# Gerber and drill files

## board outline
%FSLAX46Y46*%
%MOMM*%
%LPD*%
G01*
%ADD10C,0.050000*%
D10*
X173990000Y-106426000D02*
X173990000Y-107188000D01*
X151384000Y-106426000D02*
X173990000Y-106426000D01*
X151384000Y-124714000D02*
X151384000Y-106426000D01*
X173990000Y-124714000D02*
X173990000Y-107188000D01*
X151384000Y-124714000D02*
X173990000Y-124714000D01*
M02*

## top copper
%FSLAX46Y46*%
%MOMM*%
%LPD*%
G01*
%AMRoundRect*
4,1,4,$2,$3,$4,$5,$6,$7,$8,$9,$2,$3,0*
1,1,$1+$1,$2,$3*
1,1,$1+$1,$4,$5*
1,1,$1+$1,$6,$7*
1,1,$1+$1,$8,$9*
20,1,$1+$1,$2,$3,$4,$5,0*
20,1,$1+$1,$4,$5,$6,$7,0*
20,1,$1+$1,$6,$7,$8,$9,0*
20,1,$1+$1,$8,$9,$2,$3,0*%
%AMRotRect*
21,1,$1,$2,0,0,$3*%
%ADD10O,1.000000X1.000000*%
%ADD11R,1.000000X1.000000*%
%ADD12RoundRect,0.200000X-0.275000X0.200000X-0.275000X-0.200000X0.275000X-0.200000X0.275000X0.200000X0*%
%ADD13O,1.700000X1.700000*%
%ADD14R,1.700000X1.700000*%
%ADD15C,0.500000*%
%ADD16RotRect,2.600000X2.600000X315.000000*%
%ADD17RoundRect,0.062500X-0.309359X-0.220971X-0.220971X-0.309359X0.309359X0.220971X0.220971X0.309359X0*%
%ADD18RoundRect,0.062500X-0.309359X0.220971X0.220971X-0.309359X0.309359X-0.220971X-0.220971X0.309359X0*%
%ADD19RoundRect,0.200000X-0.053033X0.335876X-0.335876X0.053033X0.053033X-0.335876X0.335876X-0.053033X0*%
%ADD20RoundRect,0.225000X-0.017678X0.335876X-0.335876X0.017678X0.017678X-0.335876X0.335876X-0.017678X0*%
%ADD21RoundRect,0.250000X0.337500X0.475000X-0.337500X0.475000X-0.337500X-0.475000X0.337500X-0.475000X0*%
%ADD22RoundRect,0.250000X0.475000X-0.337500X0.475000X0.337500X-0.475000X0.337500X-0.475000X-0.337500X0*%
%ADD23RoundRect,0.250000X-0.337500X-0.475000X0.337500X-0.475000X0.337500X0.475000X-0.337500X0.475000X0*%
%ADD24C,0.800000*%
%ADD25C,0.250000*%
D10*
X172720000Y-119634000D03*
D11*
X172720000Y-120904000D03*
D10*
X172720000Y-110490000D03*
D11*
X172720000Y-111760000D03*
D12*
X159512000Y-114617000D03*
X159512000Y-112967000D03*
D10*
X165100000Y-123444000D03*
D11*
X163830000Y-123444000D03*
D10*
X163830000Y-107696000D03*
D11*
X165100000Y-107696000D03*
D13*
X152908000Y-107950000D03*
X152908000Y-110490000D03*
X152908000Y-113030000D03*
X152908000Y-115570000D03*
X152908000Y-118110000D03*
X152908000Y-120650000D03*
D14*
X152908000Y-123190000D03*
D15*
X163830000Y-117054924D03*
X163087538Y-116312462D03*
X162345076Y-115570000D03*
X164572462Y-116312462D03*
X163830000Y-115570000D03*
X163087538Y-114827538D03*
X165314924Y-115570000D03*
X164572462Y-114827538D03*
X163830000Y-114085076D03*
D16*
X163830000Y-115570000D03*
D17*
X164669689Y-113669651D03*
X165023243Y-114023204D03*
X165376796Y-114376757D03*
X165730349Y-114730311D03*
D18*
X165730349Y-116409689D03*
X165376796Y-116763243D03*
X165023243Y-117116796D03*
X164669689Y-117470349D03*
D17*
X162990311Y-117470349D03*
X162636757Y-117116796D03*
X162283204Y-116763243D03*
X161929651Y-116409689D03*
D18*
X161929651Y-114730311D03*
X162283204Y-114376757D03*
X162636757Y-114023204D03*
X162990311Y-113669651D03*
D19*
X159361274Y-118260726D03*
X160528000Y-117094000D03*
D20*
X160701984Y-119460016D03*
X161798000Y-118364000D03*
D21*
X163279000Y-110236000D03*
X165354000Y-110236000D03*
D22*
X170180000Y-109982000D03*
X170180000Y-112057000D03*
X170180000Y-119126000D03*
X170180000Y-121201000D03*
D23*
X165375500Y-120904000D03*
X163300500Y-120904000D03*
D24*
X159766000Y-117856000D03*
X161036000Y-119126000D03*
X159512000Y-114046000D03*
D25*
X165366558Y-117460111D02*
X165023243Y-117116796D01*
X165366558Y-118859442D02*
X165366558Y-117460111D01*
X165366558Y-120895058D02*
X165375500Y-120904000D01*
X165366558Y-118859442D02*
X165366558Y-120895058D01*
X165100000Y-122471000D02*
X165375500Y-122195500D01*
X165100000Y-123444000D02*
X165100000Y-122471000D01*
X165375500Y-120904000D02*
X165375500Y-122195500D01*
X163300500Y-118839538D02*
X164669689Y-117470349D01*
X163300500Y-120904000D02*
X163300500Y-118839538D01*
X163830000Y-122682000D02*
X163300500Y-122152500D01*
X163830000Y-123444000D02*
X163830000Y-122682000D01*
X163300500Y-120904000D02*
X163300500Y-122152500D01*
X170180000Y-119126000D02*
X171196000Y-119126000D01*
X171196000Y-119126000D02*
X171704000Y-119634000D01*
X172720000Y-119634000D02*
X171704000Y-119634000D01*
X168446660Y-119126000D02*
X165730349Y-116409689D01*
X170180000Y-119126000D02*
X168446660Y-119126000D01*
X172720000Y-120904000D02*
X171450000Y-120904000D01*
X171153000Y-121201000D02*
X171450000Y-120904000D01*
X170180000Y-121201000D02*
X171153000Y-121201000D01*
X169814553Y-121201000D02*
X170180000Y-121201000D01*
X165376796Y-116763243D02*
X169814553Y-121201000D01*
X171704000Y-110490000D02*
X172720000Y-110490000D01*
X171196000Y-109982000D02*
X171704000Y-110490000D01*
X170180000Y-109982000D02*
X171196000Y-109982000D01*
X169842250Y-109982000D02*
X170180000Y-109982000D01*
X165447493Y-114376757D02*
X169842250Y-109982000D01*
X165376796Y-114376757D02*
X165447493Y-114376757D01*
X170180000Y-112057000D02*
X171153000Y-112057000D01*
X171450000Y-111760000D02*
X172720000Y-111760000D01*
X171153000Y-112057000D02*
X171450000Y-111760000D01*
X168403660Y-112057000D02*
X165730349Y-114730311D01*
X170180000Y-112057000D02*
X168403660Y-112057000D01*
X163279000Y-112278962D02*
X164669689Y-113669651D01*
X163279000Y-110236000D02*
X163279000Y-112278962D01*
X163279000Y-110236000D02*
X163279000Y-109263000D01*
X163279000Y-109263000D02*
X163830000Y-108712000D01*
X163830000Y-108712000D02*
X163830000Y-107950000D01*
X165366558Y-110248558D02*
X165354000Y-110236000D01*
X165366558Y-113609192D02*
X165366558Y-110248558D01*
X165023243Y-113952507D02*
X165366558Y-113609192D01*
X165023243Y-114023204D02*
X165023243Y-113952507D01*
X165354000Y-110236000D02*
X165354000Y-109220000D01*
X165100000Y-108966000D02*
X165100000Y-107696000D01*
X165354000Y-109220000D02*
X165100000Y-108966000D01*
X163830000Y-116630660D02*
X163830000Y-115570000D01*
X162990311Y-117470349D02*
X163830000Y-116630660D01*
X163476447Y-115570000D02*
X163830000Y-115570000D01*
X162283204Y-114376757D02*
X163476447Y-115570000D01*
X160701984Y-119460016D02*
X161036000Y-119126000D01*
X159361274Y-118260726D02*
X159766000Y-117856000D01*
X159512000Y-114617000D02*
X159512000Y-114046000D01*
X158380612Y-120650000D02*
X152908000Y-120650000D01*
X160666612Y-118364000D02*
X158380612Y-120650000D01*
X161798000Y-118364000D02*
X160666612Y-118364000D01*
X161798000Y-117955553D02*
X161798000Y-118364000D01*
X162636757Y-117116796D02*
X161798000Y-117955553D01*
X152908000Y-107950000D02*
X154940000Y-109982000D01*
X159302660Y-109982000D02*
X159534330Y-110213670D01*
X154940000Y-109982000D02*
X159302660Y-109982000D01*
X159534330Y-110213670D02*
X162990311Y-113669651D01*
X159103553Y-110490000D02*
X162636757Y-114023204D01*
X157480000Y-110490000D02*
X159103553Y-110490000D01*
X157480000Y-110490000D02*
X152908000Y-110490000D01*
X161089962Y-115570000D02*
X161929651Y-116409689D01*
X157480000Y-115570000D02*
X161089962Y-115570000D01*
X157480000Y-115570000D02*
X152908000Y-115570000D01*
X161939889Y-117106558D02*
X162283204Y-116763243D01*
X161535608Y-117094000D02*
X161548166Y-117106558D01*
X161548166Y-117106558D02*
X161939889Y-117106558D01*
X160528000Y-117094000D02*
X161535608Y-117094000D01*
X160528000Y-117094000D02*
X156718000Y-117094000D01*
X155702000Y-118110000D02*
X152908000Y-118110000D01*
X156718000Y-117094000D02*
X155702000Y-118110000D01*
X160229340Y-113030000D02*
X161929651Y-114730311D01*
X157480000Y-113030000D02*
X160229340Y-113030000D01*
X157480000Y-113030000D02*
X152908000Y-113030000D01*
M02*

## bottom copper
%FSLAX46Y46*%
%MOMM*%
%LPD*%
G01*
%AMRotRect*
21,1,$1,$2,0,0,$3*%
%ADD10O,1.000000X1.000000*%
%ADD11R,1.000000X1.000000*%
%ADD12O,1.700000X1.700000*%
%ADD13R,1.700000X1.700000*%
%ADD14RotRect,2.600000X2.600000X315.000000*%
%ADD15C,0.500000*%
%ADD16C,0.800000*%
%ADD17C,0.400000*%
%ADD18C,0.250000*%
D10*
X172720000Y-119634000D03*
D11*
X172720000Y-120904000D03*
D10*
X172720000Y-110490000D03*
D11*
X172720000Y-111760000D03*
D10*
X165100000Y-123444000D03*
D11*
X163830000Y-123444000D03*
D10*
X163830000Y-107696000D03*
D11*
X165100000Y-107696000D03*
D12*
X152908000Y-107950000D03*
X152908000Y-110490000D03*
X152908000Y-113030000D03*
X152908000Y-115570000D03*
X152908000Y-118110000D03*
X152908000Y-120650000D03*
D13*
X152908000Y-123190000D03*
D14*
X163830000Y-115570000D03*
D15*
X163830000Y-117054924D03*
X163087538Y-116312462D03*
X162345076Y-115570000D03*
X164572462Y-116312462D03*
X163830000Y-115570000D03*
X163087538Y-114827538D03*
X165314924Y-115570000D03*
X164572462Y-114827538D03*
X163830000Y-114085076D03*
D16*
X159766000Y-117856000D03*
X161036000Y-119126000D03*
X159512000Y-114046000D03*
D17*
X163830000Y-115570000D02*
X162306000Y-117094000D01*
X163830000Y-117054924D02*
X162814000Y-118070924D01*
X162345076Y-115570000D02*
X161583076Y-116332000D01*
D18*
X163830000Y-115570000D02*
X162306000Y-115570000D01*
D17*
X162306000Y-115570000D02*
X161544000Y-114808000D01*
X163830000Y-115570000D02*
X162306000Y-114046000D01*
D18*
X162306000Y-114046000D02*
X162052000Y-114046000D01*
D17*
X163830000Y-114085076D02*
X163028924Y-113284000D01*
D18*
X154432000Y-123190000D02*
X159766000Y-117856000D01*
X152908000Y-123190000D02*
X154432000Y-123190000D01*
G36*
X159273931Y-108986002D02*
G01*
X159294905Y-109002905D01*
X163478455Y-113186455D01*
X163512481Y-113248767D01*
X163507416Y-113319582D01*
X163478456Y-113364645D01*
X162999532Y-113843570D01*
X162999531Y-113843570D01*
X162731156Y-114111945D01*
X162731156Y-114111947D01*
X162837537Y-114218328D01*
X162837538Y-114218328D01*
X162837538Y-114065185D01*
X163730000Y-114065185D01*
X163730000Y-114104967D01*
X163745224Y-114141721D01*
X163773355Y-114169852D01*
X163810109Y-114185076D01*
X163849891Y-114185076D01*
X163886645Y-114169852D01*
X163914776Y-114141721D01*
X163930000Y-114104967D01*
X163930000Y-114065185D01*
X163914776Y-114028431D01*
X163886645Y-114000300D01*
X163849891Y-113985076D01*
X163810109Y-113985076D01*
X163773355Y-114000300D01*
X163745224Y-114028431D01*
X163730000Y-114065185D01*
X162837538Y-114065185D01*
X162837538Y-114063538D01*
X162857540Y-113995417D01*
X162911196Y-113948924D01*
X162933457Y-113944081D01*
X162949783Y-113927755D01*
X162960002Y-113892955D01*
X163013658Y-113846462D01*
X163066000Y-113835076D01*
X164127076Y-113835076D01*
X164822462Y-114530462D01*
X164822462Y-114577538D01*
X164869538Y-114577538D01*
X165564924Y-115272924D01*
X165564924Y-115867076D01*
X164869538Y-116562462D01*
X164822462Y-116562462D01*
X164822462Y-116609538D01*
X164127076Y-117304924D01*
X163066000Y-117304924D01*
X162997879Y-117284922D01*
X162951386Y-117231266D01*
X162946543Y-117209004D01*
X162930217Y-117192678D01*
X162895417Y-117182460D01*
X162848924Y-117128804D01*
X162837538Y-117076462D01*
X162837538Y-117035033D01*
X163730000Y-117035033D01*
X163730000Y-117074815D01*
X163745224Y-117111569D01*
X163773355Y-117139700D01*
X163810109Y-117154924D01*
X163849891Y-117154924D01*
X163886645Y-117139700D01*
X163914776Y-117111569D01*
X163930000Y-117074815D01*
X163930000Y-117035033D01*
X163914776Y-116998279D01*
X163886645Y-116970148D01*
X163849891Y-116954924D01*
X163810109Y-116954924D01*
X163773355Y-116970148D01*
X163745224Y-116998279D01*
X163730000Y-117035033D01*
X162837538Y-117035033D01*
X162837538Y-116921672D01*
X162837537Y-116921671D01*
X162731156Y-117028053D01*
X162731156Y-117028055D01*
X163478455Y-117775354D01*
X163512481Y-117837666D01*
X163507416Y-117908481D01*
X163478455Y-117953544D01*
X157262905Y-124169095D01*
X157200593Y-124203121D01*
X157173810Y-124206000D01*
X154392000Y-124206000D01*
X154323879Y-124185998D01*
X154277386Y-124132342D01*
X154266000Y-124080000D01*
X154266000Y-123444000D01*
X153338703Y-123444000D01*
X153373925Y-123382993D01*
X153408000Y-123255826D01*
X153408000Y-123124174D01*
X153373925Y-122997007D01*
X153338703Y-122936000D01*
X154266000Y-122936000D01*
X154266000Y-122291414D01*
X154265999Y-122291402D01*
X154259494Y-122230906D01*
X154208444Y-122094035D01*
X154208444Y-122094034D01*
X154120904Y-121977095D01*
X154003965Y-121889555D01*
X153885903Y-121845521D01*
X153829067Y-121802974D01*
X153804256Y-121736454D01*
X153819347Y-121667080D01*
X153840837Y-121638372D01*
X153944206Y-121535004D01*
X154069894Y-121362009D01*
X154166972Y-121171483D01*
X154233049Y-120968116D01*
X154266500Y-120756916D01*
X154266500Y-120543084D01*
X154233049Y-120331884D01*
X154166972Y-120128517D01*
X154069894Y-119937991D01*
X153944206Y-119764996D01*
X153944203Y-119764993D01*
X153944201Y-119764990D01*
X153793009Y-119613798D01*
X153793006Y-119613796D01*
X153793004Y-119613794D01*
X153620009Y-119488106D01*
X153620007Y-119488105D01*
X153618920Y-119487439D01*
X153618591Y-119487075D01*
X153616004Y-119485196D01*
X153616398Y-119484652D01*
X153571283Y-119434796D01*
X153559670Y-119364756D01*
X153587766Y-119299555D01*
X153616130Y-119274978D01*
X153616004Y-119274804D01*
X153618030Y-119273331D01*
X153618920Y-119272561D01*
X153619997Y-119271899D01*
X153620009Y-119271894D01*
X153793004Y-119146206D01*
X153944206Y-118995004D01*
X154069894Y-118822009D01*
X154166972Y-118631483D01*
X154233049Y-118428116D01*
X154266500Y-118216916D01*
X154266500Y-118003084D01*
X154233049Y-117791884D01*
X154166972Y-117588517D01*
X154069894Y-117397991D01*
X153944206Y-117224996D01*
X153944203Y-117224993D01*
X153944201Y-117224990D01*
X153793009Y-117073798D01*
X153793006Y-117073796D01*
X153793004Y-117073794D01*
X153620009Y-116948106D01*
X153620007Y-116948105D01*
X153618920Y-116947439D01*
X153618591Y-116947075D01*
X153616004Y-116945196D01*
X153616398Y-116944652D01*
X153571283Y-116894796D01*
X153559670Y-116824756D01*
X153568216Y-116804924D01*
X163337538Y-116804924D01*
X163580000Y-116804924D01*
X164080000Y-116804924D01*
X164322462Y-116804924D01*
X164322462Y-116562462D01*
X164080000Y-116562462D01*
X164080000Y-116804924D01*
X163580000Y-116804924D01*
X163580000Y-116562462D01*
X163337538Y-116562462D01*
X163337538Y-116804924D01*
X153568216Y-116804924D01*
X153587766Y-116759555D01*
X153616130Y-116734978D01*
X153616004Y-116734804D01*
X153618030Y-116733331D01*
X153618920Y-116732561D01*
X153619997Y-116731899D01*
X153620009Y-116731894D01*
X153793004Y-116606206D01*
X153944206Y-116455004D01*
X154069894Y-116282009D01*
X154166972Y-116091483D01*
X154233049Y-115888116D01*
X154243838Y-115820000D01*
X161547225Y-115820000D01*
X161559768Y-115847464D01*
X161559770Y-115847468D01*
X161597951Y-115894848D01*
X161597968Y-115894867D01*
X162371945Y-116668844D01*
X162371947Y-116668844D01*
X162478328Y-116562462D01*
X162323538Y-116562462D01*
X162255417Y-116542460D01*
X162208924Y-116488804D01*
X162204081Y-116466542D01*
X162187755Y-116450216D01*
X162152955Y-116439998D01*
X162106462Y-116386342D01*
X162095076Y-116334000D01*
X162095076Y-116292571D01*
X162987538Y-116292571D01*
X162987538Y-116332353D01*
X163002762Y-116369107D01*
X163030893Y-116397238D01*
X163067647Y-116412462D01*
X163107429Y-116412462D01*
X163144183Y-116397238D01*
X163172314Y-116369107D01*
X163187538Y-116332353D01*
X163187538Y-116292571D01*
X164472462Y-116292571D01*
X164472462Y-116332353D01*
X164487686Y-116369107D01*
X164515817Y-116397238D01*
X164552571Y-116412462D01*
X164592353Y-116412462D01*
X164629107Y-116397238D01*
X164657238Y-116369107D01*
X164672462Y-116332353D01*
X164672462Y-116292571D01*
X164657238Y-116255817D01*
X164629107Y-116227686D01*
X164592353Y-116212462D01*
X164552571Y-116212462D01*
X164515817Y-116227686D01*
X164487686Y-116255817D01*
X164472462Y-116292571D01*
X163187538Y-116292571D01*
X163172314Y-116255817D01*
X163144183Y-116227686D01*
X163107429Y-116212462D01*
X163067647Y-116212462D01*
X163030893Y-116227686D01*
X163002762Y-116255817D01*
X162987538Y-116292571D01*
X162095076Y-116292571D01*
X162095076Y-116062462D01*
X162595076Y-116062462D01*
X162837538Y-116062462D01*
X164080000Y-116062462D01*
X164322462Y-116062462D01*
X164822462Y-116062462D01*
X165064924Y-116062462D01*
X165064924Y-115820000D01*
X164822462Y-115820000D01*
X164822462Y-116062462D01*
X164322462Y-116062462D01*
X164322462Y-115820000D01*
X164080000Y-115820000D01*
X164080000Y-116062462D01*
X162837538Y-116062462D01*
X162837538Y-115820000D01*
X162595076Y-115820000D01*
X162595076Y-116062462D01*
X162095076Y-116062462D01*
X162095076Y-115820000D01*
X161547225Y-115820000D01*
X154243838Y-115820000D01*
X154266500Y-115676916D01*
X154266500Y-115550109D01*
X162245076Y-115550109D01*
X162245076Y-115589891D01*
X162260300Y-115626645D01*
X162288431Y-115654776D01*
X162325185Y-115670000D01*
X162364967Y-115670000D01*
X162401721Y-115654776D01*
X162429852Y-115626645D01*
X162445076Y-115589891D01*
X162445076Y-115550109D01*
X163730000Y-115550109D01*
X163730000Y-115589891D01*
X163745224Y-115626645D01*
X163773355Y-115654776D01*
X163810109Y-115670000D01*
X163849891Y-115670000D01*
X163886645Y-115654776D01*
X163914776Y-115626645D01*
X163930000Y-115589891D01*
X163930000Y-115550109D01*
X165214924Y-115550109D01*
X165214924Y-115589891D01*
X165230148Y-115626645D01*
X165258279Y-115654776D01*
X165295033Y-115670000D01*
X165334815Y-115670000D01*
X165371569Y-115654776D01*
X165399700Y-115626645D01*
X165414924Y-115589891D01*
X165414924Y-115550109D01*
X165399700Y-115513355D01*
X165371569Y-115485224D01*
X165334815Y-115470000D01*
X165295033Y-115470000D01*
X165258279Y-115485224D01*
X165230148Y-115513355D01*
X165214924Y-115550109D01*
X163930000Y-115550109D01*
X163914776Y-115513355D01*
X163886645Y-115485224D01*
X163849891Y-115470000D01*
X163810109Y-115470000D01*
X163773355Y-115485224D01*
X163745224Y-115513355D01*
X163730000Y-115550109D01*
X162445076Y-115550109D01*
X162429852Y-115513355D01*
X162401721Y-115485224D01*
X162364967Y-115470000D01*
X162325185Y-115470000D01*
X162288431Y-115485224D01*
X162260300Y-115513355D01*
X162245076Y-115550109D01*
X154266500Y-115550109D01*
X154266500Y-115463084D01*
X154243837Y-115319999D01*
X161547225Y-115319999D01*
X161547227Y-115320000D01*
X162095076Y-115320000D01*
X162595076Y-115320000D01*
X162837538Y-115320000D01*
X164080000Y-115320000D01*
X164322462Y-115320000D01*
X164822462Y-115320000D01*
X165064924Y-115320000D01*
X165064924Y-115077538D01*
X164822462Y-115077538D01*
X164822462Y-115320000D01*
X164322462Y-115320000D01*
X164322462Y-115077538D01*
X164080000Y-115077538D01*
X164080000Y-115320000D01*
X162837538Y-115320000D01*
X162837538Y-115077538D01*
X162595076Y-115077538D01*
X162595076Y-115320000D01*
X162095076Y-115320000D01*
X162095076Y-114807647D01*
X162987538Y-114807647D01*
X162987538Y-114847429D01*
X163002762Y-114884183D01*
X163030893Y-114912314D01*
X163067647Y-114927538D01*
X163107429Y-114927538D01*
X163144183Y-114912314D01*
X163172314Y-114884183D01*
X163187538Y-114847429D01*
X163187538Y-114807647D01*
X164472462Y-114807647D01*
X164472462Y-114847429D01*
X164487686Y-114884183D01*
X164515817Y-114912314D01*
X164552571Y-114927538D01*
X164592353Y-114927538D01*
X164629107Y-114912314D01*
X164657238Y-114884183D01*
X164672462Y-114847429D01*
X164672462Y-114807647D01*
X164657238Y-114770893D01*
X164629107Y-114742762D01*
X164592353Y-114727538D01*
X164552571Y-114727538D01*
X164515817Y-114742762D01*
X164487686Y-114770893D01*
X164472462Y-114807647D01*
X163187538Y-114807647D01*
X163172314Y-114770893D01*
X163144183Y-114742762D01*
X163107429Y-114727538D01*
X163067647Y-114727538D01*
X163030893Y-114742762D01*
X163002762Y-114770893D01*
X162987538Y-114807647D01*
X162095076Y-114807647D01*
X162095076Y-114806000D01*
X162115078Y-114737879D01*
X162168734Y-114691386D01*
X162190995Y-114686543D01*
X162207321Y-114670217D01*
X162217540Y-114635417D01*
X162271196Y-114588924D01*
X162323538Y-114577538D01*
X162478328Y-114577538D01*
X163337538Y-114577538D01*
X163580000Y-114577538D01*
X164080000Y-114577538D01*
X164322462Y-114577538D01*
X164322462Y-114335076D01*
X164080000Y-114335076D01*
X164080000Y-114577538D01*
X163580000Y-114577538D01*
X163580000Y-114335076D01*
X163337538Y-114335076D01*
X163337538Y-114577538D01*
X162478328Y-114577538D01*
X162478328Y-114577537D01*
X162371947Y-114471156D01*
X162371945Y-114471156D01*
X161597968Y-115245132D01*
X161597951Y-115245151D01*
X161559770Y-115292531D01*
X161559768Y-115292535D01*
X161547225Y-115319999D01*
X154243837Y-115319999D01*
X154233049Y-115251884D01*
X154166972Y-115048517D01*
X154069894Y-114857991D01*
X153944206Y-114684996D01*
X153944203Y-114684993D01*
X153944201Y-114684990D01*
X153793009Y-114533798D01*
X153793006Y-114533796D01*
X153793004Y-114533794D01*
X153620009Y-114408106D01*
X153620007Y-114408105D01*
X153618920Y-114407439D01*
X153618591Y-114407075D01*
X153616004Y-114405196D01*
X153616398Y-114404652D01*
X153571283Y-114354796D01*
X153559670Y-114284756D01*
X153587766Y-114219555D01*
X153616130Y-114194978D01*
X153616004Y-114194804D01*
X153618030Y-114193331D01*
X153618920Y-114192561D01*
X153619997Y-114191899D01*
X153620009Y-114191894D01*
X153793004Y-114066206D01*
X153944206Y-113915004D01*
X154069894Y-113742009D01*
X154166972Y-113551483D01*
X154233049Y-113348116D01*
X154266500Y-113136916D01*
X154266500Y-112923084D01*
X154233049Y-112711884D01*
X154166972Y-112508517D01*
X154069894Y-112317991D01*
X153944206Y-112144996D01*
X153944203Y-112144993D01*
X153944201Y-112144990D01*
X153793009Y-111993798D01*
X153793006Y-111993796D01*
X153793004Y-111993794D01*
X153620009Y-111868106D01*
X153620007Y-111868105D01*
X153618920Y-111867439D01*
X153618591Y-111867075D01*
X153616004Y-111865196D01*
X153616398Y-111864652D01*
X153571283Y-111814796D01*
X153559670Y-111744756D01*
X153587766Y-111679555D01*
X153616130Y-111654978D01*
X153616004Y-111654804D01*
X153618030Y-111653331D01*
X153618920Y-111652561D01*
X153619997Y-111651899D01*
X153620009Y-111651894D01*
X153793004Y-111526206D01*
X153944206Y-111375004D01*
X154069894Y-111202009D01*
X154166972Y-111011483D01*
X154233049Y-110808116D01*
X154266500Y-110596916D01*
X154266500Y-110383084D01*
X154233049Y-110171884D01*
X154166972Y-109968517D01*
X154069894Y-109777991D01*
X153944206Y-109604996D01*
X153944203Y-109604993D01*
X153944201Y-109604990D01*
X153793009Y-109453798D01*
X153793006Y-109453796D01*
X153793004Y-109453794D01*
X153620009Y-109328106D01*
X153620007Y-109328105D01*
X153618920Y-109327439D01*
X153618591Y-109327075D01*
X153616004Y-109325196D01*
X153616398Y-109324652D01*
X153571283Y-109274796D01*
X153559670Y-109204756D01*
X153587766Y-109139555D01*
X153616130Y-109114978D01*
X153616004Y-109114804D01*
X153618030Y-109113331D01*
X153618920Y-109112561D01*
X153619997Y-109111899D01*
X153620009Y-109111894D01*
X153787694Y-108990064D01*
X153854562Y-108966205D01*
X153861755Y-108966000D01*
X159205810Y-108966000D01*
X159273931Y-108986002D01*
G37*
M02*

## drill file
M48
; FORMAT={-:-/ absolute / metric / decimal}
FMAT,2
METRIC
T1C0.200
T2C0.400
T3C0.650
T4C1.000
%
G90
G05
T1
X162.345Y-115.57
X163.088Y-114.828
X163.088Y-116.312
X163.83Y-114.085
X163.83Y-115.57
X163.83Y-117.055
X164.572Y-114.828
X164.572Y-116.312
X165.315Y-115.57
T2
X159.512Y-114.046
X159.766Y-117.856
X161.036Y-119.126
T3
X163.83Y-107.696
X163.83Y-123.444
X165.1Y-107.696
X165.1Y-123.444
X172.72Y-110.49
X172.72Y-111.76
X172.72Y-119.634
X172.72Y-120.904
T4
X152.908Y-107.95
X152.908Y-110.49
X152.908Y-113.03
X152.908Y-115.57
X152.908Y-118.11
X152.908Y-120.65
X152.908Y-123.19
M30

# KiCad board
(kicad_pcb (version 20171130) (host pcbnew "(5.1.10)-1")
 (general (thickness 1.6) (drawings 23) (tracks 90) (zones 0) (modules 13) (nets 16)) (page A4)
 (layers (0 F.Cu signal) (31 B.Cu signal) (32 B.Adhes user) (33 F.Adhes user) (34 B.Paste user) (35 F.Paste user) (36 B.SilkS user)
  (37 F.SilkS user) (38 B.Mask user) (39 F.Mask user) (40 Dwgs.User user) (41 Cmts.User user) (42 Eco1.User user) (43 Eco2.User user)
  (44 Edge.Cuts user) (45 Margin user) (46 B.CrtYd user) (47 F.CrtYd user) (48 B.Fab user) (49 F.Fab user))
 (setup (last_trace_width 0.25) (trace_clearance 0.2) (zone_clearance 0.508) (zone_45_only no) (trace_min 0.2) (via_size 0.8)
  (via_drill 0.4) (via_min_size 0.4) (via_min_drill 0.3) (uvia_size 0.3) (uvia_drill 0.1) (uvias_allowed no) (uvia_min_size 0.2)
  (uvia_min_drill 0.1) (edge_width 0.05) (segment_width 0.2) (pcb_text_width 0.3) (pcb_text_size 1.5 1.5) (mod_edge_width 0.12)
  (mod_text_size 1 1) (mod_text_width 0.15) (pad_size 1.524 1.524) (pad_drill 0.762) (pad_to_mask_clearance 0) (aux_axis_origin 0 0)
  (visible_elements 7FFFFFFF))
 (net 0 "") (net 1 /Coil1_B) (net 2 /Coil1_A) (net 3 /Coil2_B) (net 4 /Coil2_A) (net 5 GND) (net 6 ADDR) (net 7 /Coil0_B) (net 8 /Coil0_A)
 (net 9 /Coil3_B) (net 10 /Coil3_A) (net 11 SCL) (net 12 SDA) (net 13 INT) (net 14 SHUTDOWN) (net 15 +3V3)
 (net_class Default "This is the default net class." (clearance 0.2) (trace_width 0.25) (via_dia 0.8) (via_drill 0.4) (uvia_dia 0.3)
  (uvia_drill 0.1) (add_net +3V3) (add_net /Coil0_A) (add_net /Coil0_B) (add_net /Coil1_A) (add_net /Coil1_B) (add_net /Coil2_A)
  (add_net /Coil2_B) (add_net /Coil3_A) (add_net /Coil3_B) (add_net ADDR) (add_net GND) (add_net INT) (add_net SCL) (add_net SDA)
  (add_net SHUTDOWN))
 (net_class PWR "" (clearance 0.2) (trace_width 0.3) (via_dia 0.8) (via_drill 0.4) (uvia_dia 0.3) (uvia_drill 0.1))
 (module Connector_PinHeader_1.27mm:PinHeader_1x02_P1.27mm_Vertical (layer F.Cu) (at 172.72 120.904 180)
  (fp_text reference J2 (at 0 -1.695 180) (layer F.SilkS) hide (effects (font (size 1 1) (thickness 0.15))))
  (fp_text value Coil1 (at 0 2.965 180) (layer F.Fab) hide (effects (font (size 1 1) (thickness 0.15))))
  (pad 2 thru_hole oval (at 0 1.27 180) (size 1 1) (drill 0.65) (layers *.Cu *.Mask) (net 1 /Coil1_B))
  (pad 1 thru_hole rect (at 0 0 180) (size 1 1) (drill 0.65) (layers *.Cu *.Mask) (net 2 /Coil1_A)))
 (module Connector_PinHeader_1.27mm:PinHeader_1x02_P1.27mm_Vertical (layer F.Cu) (at 172.72 111.76 180)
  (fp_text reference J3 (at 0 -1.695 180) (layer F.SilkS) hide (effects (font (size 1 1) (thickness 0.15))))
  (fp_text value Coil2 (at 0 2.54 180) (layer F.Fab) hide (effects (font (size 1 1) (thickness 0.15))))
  (pad 2 thru_hole oval (at 0 1.27 180) (size 1 1) (drill 0.65) (layers *.Cu *.Mask) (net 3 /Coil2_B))
  (pad 1 thru_hole rect (at 0 0 180) (size 1 1) (drill 0.65) (layers *.Cu *.Mask) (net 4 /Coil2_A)))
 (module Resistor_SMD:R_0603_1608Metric (layer F.Cu) (at 159.512 113.792 270)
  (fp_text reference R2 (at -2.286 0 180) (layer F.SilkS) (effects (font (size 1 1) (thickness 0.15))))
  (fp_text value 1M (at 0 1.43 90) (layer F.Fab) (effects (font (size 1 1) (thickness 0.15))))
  (pad 2 smd roundrect (at 0.825 0 270) (size 0.8 0.95) (layers F.Cu F.Paste F.Mask) (roundrect_rratio 0.25) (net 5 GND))
  (pad 1 smd roundrect (at -0.825 0 270) (size 0.8 0.95) (layers F.Cu F.Paste F.Mask) (roundrect_rratio 0.25) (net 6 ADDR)))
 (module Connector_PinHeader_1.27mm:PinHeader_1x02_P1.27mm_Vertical (layer F.Cu) (at 163.83 123.444 90)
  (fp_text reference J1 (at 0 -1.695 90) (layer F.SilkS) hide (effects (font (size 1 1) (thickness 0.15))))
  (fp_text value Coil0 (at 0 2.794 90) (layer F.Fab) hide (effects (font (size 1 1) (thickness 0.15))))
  (pad 2 thru_hole oval (at 0 1.27 90) (size 1 1) (drill 0.65) (layers *.Cu *.Mask) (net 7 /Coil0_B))
  (pad 1 thru_hole rect (at 0 0 90) (size 1 1) (drill 0.65) (layers *.Cu *.Mask) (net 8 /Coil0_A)))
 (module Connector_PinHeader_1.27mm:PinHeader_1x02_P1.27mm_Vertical (layer F.Cu) (at 165.1 107.696 270)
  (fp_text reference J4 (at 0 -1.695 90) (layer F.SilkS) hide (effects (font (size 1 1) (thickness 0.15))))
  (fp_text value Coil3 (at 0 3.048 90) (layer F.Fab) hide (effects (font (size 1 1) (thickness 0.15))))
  (pad 2 thru_hole oval (at 0 1.27 270) (size 1 1) (drill 0.65) (layers *.Cu *.Mask) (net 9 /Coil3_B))
  (pad 1 thru_hole rect (at 0 0 270) (size 1 1) (drill 0.65) (layers *.Cu *.Mask) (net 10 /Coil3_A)))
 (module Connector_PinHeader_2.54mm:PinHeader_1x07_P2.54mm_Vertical (layer F.Cu) (at 152.908 123.19 180)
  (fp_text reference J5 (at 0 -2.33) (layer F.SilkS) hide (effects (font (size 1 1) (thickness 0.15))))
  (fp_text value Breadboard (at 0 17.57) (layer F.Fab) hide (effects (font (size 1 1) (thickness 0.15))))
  (pad 7 thru_hole oval (at 0 15.24 180) (size 1.7 1.7) (drill 1) (layers *.Cu *.Mask) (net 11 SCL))
  (pad 6 thru_hole oval (at 0 12.7 180) (size 1.7 1.7) (drill 1) (layers *.Cu *.Mask) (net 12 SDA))
  (pad 5 thru_hole oval (at 0 10.16 180) (size 1.7 1.7) (drill 1) (layers *.Cu *.Mask) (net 6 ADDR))
  (pad 4 thru_hole oval (at 0 7.62 180) (size 1.7 1.7) (drill 1) (layers *.Cu *.Mask) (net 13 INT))
  (pad 3 thru_hole oval (at 0 5.08 180) (size 1.7 1.7) (drill 1) (layers *.Cu *.Mask) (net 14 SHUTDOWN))
  (pad 2 thru_hole oval (at 0 2.54 180) (size 1.7 1.7) (drill 1) (layers *.Cu *.Mask) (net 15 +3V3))
  (pad 1 thru_hole rect (at 0 0 180) (size 1.7 1.7) (drill 1) (layers *.Cu *.Mask) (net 5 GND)))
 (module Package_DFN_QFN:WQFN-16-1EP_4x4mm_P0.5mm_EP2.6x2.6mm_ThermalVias (layer F.Cu) (at 163.83 115.57 315)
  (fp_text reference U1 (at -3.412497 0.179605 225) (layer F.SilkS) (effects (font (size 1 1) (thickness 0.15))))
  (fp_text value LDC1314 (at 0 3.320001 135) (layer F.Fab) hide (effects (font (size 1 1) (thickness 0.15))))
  (pad "" smd roundrect (at 0.65 0.65 315) (size 1.13 1.13) (layers F.Paste) (roundrect_rratio 0.2212389380530974))
  (pad "" smd roundrect (at 0.65 -0.65 315) (size 1.13 1.13) (layers F.Paste) (roundrect_rratio 0.2212389380530974))
  (pad "" smd roundrect (at -0.65 0.65 315) (size 1.13 1.13) (layers F.Paste) (roundrect_rratio 0.2212389380530974))
  (pad "" smd roundrect (at -0.65 -0.65 315) (size 1.13 1.13) (layers F.Paste) (roundrect_rratio 0.2212389380530974))
  (pad 17 smd rect (at 0 0 315) (size 2.6 2.6) (layers B.Cu) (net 5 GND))
  (pad 17 thru_hole circle (at 1.05 1.05 315) (size 0.5 0.5) (drill 0.2) (layers *.Cu) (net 5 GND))
  (pad 17 thru_hole circle (at 0 1.05 315) (size 0.5 0.5) (drill 0.2) (layers *.Cu) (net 5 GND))
  (pad 17 thru_hole circle (at -1.05 1.05 315) (size 0.5 0.5) (drill 0.2) (layers *.Cu) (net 5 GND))
  (pad 17 thru_hole circle (at 1.05 0 315) (size 0.5 0.5) (drill 0.2) (layers *.Cu) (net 5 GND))
  (pad 17 thru_hole circle (at 0 0 315) (size 0.5 0.5) (drill 0.2) (layers *.Cu) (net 5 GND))
  (pad 17 thru_hole circle (at -1.05 0 315) (size 0.5 0.5) (drill 0.2) (layers *.Cu) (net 5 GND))
  (pad 17 thru_hole circle (at 1.05 -1.05 315) (size 0.5 0.5) (drill 0.2) (layers *.Cu) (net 5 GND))
  (pad 17 thru_hole circle (at 0 -1.05 315) (size 0.5 0.5) (drill 0.2) (layers *.Cu) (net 5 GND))
  (pad 17 thru_hole circle (at -1.05 -1.05 315) (size 0.5 0.5) (drill 0.2) (layers *.Cu) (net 5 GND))
  (pad 17 smd rect (at 0 0 315) (size 2.6 2.6) (layers F.Cu F.Mask) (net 5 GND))
  (pad 16 smd roundrect (at -0.75 -1.9375 315) (size 0.25 0.875) (layers F.Cu F.Paste F.Mask) (roundrect_rratio 0.25) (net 9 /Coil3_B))
  (pad 15 smd roundrect (at -0.25 -1.9375 315) (size 0.25 0.875) (layers F.Cu F.Paste F.Mask) (roundrect_rratio 0.25) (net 10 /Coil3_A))
  (pad 14 smd roundrect (at 0.25 -1.9375 315) (size 0.25 0.875) (layers F.Cu F.Paste F.Mask) (roundrect_rratio 0.25) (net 3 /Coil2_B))
  (pad 13 smd roundrect (at 0.75 -1.9375 315) (size 0.25 0.875) (layers F.Cu F.Paste F.Mask) (roundrect_rratio 0.25) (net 4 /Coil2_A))
  (pad 12 smd roundrect (at 1.9375 -0.75 315) (size 0.875 0.25) (layers F.Cu F.Paste F.Mask) (roundrect_rratio 0.25) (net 1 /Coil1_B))
  (pad 11 smd roundrect (at 1.9375 -0.25 315) (size 0.875 0.25) (layers F.Cu F.Paste F.Mask) (roundrect_rratio 0.25) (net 2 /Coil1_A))
  (pad 10 smd roundrect (at 1.9375 0.25 315) (size 0.875 0.25) (layers F.Cu F.Paste F.Mask) (roundrect_rratio 0.25) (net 7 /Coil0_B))
  (pad 9 smd roundrect (at 1.9375 0.75 315) (size 0.875 0.25) (layers F.Cu F.Paste F.Mask) (roundrect_rratio 0.25) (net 8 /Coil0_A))
  (pad 8 smd roundrect (at 0.75 1.9375 315) (size 0.25 0.875) (layers F.Cu F.Paste F.Mask) (roundrect_rratio 0.25) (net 5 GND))
  (pad 7 smd roundrect (at 0.25 1.9375 315) (size 0.25 0.875) (layers F.Cu F.Paste F.Mask) (roundrect_rratio 0.25) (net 15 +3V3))
  (pad 6 smd roundrect (at -0.25 1.9375 315) (size 0.25 0.875) (layers F.Cu F.Paste F.Mask) (roundrect_rratio 0.25) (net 14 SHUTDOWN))
  (pad 5 smd roundrect (at -0.75 1.9375 315) (size 0.25 0.875) (layers F.Cu F.Paste F.Mask) (roundrect_rratio 0.25) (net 13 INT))
  (pad 4 smd roundrect (at -1.9375 0.75 315) (size 0.875 0.25) (layers F.Cu F.Paste F.Mask) (roundrect_rratio 0.25) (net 6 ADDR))
  (pad 3 smd roundrect (at -1.9375 0.25 315) (size 0.875 0.25) (layers F.Cu F.Paste F.Mask) (roundrect_rratio 0.25) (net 5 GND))
  (pad 2 smd roundrect (at -1.9375 -0.25 315) (size 0.875 0.25) (layers F.Cu F.Paste F.Mask) (roundrect_rratio 0.25) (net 12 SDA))
  (pad 1 smd roundrect (at -1.9375 -0.75 315) (size 0.875 0.25) (layers F.Cu F.Paste F.Mask) (roundrect_rratio 0.25) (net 11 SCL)))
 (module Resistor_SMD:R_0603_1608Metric (layer F.Cu) (at 159.944637 117.677363 225)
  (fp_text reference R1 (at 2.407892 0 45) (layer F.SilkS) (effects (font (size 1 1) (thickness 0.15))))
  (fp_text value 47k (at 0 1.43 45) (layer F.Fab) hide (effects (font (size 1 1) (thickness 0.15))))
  (pad 2 smd roundrect (at 0.825 0 225) (size 0.8 0.95) (layers F.Cu F.Paste F.Mask) (roundrect_rratio 0.25) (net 5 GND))
  (pad 1 smd roundrect (at -0.825 0 225) (size 0.8 0.95) (layers F.Cu F.Paste F.Mask) (roundrect_rratio 0.25) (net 14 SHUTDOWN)))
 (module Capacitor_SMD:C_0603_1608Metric (layer F.Cu) (at 161.249992 118.912008 225)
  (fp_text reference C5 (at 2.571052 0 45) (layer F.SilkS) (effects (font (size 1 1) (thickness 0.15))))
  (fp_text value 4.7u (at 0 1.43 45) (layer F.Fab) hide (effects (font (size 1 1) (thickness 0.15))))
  (pad 2 smd roundrect (at 0.775 0 225) (size 0.9 0.95) (layers F.Cu F.Paste F.Mask) (roundrect_rratio 0.25) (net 5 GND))
  (pad 1 smd roundrect (at -0.775 0 225) (size 0.9 0.95) (layers F.Cu F.Paste F.Mask) (roundrect_rratio 0.25) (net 15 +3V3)))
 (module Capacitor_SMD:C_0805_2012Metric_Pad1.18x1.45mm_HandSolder (layer F.Cu) (at 164.3165 110.236 180)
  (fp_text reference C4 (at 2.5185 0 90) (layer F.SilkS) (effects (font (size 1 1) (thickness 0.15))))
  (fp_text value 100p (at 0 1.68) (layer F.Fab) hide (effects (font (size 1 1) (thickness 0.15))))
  (pad 2 smd roundrect (at 1.0375 0 180) (size 1.175 1.45) (layers F.Cu F.Paste F.Mask) (roundrect_rratio 0.2127659574468085)
   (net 9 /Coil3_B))
  (pad 1 smd roundrect (at -1.0375 0 180) (size 1.175 1.45) (layers F.Cu F.Paste F.Mask) (roundrect_rratio 0.2127659574468085)
   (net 10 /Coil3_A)))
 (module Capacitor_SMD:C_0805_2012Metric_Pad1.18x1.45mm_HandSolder (layer F.Cu) (at 170.18 111.0195 90)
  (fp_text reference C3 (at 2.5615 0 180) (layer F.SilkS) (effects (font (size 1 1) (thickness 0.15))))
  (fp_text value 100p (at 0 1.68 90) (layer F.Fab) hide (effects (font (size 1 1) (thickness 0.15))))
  (pad 2 smd roundrect (at 1.0375 0 90) (size 1.175 1.45) (layers F.Cu F.Paste F.Mask) (roundrect_rratio 0.2127659574468085)
   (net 3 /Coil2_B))
  (pad 1 smd roundrect (at -1.0375 0 90) (size 1.175 1.45) (layers F.Cu F.Paste F.Mask) (roundrect_rratio 0.2127659574468085)
   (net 4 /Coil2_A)))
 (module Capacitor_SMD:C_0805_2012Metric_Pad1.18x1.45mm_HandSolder (layer F.Cu) (at 170.18 120.1635 90)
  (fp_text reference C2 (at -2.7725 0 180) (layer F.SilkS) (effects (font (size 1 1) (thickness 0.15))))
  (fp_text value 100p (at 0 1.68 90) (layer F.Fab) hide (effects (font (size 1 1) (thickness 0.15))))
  (pad 2 smd roundrect (at 1.0375 0 90) (size 1.175 1.45) (layers F.Cu F.Paste F.Mask) (roundrect_rratio 0.2127659574468085)
   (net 1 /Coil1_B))
  (pad 1 smd roundrect (at -1.0375 0 90) (size 1.175 1.45) (layers F.Cu F.Paste F.Mask) (roundrect_rratio 0.2127659574468085)
   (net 2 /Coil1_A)))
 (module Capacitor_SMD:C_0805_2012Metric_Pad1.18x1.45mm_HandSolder (layer F.Cu) (at 164.338 120.904)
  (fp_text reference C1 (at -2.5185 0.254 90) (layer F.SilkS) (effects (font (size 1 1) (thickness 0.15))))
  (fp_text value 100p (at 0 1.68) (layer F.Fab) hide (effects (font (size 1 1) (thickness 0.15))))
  (pad 2 smd roundrect (at 1.0375 0) (size 1.175 1.45) (layers F.Cu F.Paste F.Mask) (roundrect_rratio 0.2127659574468085) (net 7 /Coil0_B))
  (pad 1 smd roundrect (at -1.0375 0) (size 1.175 1.45) (layers F.Cu F.Paste F.Mask) (roundrect_rratio 0.2127659574468085) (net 8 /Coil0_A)))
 (gr_line (start 173.99 106.426) (end 173.99 107.188) (layer Edge.Cuts) (width 0.05))
 (gr_line (start 151.384 106.426) (end 173.99 106.426) (layer Edge.Cuts) (width 0.05))
 (gr_line (start 151.384 124.714) (end 151.384 106.426) (layer Edge.Cuts) (width 0.05))
 (gr_line (start 173.99 124.714) (end 173.99 107.188) (layer Edge.Cuts) (width 0.05))
 (gr_line (start 151.384 124.714) (end 173.99 124.714) (layer Edge.Cuts) (width 0.05))
 (segment (start 165.366558 117.460111) (end 165.023243 117.116796) (width 0.25) (layer F.Cu) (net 7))
 (segment (start 165.366558 118.859442) (end 165.366558 117.460111) (width 0.25) (layer F.Cu) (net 7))
 (segment (start 165.366558 120.895058) (end 165.3755 120.904) (width 0.25) (layer F.Cu) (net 7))
 (segment (start 165.366558 118.859442) (end 165.366558 120.895058) (width 0.25) (layer F.Cu) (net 7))
 (segment (start 165.1 122.471) (end 165.3755 122.1955) (width 0.25) (layer F.Cu) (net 7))
 (segment (start 165.1 123.444) (end 165.1 122.471) (width 0.25) (layer F.Cu) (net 7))
 (segment (start 165.3755 120.904) (end 165.3755 122.1955) (width 0.25) (layer F.Cu) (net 7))
 (segment (start 163.3005 118.839538) (end 164.669689 117.470349) (width 0.25) (layer F.Cu) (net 8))
 (segment (start 163.3005 120.904) (end 163.3005 118.839538) (width 0.25) (layer F.Cu) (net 8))
 (segment (start 163.83 122.682) (end 163.3005 122.1525) (width 0.25) (layer F.Cu) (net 8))
 (segment (start 163.83 123.444) (end 163.83 122.682) (width 0.25) (layer F.Cu) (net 8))
 (segment (start 163.3005 120.904) (end 163.3005 122.1525) (width 0.25) (layer F.Cu) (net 8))
 (segment (start 170.18 119.126) (end 171.196 119.126) (width 0.25) (layer F.Cu) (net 1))
 (segment (start 171.196 119.126) (end 171.704 119.634) (width 0.25) (layer F.Cu) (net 1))
 (segment (start 172.72 119.634) (end 171.704 119.634) (width 0.25) (layer F.Cu) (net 1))
 (segment (start 168.44666 119.126) (end 165.730349 116.409689) (width 0.25) (layer F.Cu) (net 1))
 (segment (start 170.18 119.126) (end 168.44666 119.126) (width 0.25) (layer F.Cu) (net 1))
 (segment (start 172.72 120.904) (end 171.45 120.904) (width 0.25) (layer F.Cu) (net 2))
 (segment (start 171.153 121.201) (end 171.45 120.904) (width 0.25) (layer F.Cu) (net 2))
 (segment (start 170.18 121.201) (end 171.153 121.201) (width 0.25) (layer F.Cu) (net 2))
 (segment (start 169.814553 121.201) (end 170.18 121.201) (width 0.25) (layer F.Cu) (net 2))
 (segment (start 165.376796 116.763243) (end 169.814553 121.201) (width 0.25) (layer F.Cu) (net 2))
 (segment (start 171.704 110.49) (end 172.72 110.49) (width 0.25) (layer F.Cu) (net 3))
 (segment (start 171.196 109.982) (end 171.704 110.49) (width 0.25) (layer F.Cu) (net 3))
 (segment (start 170.18 109.982) (end 171.196 109.982) (width 0.25) (layer F.Cu) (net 3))
 (segment (start 169.84225 109.982) (end 170.18 109.982) (width 0.25) (layer F.Cu) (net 3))
 (segment (start 165.447493 114.376757) (end 169.84225 109.982) (width 0.25) (layer F.Cu) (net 3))
 (segment (start 165.376796 114.376757) (end 165.447493 114.376757) (width 0.25) (layer F.Cu) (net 3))
 (segment (start 170.18 112.057) (end 171.153 112.057) (width 0.25) (layer F.Cu) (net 4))
 (segment (start 171.45 111.76) (end 172.72 111.76) (width 0.25) (layer F.Cu) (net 4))
 (segment (start 171.153 112.057) (end 171.45 111.76) (width 0.25) (layer F.Cu) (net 4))
 (segment (start 168.40366 112.057) (end 165.730349 114.730311) (width 0.25) (layer F.Cu) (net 4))
 (segment (start 170.18 112.057) (end 168.40366 112.057) (width 0.25) (layer F.Cu) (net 4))
 (segment (start 163.279 112.278962) (end 164.669689 113.669651) (width 0.25) (layer F.Cu) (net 9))
 (segment (start 163.279 110.236) (end 163.279 112.278962) (width 0.25) (layer F.Cu) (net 9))
 (segment (start 163.279 110.236) (end 163.279 109.263) (width 0.25) (layer F.Cu) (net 9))
 (segment (start 163.279 109.263) (end 163.83 108.712) (width 0.25) (layer F.Cu) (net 9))
 (segment (start 163.83 108.712) (end 163.83 107.95) (width 0.25) (layer F.Cu) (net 9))
 (segment (start 165.366558 110.248558) (end 165.354 110.236) (width 0.25) (layer F.Cu) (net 10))
 (segment (start 165.366558 113.609192) (end 165.366558 110.248558) (width 0.25) (layer F.Cu) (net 10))
 (segment (start 165.023243 113.952507) (end 165.366558 113.609192) (width 0.25) (layer F.Cu) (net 10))
 (segment (start 165.023243 114.023204) (end 165.023243 113.952507) (width 0.25) (layer F.Cu) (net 10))
 (segment (start 165.354 110.236) (end 165.354 109.22) (width 0.25) (layer F.Cu) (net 10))
 (segment (start 165.1 108.966) (end 165.1 107.696) (width 0.25) (layer F.Cu) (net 10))
 (segment (start 165.354 109.22) (end 165.1 108.966) (width 0.25) (layer F.Cu) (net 10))
 (segment (start 163.83 116.63066) (end 163.83 115.57) (width 0.25) (layer F.Cu) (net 5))
 (segment (start 162.990311 117.470349) (end 163.83 116.63066) (width 0.25) (layer F.Cu) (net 5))
 (segment (start 163.476447 115.57) (end 163.83 115.57) (width 0.25) (layer F.Cu) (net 5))
 (segment (start 162.283204 114.376757) (end 163.476447 115.57) (width 0.25) (layer F.Cu) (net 5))
 (via (at 159.766 117.856) (size 0.8) (drill 0.4) (layers F.Cu B.Cu) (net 5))
 (segment (start 163.83 115.57) (end 162.306 117.094) (width 0.4) (layer B.Cu) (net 5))
 (segment (start 163.83 117.054924) (end 162.814 118.070924) (width 0.4) (layer B.Cu) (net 5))
 (segment (start 162.345076 115.57) (end 161.583076 116.332) (width 0.4) (layer B.Cu) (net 5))
 (segment (start 163.83 115.57) (end 162.306 115.57) (width 0.25) (layer B.Cu) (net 5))
 (segment (start 162.306 115.57) (end 161.544 114.808) (width 0.4) (layer B.Cu) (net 5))
 (segment (start 163.83 115.57) (end 162.306 114.046) (width 0.4) (layer B.Cu) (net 5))
 (segment (start 162.306 114.046) (end 162.052 114.046) (width 0.25) (layer B.Cu) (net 5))
 (segment (start 163.83 114.085076) (end 163.028924 113.284) (width 0.4) (layer B.Cu) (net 5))
 (via (at 161.036 119.126) (size 0.8) (drill 0.4) (layers F.Cu B.Cu) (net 5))
 (segment (start 160.701984 119.460016) (end 161.036 119.126) (width 0.25) (layer F.Cu) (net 5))
 (segment (start 159.361274 118.260726) (end 159.766 117.856) (width 0.25) (layer F.Cu) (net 5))
 (segment (start 154.432 123.19) (end 159.766 117.856) (width 0.25) (layer B.Cu) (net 5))
 (segment (start 152.908 123.19) (end 154.432 123.19) (width 0.25) (layer B.Cu) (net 5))
 (via (at 159.512 114.046) (size 0.8) (drill 0.4) (layers F.Cu B.Cu) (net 5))
 (segment (start 159.512 114.617) (end 159.512 114.046) (width 0.25) (layer F.Cu) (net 5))
 (segment (start 158.380612 120.65) (end 152.908 120.65) (width 0.25) (layer F.Cu) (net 15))
 (segment (start 160.666612 118.364) (end 158.380612 120.65) (width 0.25) (layer F.Cu) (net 15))
 (segment (start 161.798 118.364) (end 160.666612 118.364) (width 0.25) (layer F.Cu) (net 15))
 (segment (start 161.798 117.955553) (end 161.798 118.364) (width 0.25) (layer F.Cu) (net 15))
 (segment (start 162.636757 117.116796) (end 161.798 117.955553) (width 0.25) (layer F.Cu) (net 15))
 (segment (start 152.908 107.95) (end 154.94 109.982) (width 0.25) (layer F.Cu) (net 11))
 (segment (start 159.30266 109.982) (end 159.53433 110.21367) (width 0.25) (layer F.Cu) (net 11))
 (segment (start 154.94 109.982) (end 159.30266 109.982) (width 0.25) (layer F.Cu) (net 11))
 (segment (start 159.53433 110.21367) (end 162.990311 113.669651) (width 0.25) (layer F.Cu) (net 11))
 (segment (start 159.103553 110.49) (end 162.636757 114.023204) (width 0.25) (layer F.Cu) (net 12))
 (segment (start 157.48 110.49) (end 159.103553 110.49) (width 0.25) (layer F.Cu) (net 12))
 (segment (start 157.48 110.49) (end 152.908 110.49) (width 0.25) (layer F.Cu) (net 12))
 (segment (start 161.089962 115.57) (end 161.929651 116.409689) (width 0.25) (layer F.Cu) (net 13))
 (segment (start 157.48 115.57) (end 161.089962 115.57) (width 0.25) (layer F.Cu) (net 13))
 (segment (start 157.48 115.57) (end 152.908 115.57) (width 0.25) (layer F.Cu) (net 13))
 (segment (start 161.939889 117.106558) (end 162.283204 116.763243) (width 0.25) (layer F.Cu) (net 14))
 (segment (start 161.535608 117.094) (end 161.548166 117.106558) (width 0.25) (layer F.Cu) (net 14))
 (segment (start 161.548166 117.106558) (end 161.939889 117.106558) (width 0.25) (layer F.Cu) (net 14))
 (segment (start 160.528 117.094) (end 161.535608 117.094) (width 0.25) (layer F.Cu) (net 14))
 (segment (start 160.528 117.094) (end 156.718 117.094) (width 0.25) (layer F.Cu) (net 14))
 (segment (start 155.702 118.11) (end 152.908 118.11) (width 0.25) (layer F.Cu) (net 14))
 (segment (start 156.718 117.094) (end 155.702 118.11) (width 0.25) (layer F.Cu) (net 14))
 (segment (start 160.22934 113.03) (end 161.929651 114.730311) (width 0.25) (layer F.Cu) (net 6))
 (segment (start 157.48 113.03) (end 160.22934 113.03) (width 0.25) (layer F.Cu) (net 6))
 (segment (start 157.48 113.03) (end 152.908 113.03) (width 0.25) (layer F.Cu) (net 6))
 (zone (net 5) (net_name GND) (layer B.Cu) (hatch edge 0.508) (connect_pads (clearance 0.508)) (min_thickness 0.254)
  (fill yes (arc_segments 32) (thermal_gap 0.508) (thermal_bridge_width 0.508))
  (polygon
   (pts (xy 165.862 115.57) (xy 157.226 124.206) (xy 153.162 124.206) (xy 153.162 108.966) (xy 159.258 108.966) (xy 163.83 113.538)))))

